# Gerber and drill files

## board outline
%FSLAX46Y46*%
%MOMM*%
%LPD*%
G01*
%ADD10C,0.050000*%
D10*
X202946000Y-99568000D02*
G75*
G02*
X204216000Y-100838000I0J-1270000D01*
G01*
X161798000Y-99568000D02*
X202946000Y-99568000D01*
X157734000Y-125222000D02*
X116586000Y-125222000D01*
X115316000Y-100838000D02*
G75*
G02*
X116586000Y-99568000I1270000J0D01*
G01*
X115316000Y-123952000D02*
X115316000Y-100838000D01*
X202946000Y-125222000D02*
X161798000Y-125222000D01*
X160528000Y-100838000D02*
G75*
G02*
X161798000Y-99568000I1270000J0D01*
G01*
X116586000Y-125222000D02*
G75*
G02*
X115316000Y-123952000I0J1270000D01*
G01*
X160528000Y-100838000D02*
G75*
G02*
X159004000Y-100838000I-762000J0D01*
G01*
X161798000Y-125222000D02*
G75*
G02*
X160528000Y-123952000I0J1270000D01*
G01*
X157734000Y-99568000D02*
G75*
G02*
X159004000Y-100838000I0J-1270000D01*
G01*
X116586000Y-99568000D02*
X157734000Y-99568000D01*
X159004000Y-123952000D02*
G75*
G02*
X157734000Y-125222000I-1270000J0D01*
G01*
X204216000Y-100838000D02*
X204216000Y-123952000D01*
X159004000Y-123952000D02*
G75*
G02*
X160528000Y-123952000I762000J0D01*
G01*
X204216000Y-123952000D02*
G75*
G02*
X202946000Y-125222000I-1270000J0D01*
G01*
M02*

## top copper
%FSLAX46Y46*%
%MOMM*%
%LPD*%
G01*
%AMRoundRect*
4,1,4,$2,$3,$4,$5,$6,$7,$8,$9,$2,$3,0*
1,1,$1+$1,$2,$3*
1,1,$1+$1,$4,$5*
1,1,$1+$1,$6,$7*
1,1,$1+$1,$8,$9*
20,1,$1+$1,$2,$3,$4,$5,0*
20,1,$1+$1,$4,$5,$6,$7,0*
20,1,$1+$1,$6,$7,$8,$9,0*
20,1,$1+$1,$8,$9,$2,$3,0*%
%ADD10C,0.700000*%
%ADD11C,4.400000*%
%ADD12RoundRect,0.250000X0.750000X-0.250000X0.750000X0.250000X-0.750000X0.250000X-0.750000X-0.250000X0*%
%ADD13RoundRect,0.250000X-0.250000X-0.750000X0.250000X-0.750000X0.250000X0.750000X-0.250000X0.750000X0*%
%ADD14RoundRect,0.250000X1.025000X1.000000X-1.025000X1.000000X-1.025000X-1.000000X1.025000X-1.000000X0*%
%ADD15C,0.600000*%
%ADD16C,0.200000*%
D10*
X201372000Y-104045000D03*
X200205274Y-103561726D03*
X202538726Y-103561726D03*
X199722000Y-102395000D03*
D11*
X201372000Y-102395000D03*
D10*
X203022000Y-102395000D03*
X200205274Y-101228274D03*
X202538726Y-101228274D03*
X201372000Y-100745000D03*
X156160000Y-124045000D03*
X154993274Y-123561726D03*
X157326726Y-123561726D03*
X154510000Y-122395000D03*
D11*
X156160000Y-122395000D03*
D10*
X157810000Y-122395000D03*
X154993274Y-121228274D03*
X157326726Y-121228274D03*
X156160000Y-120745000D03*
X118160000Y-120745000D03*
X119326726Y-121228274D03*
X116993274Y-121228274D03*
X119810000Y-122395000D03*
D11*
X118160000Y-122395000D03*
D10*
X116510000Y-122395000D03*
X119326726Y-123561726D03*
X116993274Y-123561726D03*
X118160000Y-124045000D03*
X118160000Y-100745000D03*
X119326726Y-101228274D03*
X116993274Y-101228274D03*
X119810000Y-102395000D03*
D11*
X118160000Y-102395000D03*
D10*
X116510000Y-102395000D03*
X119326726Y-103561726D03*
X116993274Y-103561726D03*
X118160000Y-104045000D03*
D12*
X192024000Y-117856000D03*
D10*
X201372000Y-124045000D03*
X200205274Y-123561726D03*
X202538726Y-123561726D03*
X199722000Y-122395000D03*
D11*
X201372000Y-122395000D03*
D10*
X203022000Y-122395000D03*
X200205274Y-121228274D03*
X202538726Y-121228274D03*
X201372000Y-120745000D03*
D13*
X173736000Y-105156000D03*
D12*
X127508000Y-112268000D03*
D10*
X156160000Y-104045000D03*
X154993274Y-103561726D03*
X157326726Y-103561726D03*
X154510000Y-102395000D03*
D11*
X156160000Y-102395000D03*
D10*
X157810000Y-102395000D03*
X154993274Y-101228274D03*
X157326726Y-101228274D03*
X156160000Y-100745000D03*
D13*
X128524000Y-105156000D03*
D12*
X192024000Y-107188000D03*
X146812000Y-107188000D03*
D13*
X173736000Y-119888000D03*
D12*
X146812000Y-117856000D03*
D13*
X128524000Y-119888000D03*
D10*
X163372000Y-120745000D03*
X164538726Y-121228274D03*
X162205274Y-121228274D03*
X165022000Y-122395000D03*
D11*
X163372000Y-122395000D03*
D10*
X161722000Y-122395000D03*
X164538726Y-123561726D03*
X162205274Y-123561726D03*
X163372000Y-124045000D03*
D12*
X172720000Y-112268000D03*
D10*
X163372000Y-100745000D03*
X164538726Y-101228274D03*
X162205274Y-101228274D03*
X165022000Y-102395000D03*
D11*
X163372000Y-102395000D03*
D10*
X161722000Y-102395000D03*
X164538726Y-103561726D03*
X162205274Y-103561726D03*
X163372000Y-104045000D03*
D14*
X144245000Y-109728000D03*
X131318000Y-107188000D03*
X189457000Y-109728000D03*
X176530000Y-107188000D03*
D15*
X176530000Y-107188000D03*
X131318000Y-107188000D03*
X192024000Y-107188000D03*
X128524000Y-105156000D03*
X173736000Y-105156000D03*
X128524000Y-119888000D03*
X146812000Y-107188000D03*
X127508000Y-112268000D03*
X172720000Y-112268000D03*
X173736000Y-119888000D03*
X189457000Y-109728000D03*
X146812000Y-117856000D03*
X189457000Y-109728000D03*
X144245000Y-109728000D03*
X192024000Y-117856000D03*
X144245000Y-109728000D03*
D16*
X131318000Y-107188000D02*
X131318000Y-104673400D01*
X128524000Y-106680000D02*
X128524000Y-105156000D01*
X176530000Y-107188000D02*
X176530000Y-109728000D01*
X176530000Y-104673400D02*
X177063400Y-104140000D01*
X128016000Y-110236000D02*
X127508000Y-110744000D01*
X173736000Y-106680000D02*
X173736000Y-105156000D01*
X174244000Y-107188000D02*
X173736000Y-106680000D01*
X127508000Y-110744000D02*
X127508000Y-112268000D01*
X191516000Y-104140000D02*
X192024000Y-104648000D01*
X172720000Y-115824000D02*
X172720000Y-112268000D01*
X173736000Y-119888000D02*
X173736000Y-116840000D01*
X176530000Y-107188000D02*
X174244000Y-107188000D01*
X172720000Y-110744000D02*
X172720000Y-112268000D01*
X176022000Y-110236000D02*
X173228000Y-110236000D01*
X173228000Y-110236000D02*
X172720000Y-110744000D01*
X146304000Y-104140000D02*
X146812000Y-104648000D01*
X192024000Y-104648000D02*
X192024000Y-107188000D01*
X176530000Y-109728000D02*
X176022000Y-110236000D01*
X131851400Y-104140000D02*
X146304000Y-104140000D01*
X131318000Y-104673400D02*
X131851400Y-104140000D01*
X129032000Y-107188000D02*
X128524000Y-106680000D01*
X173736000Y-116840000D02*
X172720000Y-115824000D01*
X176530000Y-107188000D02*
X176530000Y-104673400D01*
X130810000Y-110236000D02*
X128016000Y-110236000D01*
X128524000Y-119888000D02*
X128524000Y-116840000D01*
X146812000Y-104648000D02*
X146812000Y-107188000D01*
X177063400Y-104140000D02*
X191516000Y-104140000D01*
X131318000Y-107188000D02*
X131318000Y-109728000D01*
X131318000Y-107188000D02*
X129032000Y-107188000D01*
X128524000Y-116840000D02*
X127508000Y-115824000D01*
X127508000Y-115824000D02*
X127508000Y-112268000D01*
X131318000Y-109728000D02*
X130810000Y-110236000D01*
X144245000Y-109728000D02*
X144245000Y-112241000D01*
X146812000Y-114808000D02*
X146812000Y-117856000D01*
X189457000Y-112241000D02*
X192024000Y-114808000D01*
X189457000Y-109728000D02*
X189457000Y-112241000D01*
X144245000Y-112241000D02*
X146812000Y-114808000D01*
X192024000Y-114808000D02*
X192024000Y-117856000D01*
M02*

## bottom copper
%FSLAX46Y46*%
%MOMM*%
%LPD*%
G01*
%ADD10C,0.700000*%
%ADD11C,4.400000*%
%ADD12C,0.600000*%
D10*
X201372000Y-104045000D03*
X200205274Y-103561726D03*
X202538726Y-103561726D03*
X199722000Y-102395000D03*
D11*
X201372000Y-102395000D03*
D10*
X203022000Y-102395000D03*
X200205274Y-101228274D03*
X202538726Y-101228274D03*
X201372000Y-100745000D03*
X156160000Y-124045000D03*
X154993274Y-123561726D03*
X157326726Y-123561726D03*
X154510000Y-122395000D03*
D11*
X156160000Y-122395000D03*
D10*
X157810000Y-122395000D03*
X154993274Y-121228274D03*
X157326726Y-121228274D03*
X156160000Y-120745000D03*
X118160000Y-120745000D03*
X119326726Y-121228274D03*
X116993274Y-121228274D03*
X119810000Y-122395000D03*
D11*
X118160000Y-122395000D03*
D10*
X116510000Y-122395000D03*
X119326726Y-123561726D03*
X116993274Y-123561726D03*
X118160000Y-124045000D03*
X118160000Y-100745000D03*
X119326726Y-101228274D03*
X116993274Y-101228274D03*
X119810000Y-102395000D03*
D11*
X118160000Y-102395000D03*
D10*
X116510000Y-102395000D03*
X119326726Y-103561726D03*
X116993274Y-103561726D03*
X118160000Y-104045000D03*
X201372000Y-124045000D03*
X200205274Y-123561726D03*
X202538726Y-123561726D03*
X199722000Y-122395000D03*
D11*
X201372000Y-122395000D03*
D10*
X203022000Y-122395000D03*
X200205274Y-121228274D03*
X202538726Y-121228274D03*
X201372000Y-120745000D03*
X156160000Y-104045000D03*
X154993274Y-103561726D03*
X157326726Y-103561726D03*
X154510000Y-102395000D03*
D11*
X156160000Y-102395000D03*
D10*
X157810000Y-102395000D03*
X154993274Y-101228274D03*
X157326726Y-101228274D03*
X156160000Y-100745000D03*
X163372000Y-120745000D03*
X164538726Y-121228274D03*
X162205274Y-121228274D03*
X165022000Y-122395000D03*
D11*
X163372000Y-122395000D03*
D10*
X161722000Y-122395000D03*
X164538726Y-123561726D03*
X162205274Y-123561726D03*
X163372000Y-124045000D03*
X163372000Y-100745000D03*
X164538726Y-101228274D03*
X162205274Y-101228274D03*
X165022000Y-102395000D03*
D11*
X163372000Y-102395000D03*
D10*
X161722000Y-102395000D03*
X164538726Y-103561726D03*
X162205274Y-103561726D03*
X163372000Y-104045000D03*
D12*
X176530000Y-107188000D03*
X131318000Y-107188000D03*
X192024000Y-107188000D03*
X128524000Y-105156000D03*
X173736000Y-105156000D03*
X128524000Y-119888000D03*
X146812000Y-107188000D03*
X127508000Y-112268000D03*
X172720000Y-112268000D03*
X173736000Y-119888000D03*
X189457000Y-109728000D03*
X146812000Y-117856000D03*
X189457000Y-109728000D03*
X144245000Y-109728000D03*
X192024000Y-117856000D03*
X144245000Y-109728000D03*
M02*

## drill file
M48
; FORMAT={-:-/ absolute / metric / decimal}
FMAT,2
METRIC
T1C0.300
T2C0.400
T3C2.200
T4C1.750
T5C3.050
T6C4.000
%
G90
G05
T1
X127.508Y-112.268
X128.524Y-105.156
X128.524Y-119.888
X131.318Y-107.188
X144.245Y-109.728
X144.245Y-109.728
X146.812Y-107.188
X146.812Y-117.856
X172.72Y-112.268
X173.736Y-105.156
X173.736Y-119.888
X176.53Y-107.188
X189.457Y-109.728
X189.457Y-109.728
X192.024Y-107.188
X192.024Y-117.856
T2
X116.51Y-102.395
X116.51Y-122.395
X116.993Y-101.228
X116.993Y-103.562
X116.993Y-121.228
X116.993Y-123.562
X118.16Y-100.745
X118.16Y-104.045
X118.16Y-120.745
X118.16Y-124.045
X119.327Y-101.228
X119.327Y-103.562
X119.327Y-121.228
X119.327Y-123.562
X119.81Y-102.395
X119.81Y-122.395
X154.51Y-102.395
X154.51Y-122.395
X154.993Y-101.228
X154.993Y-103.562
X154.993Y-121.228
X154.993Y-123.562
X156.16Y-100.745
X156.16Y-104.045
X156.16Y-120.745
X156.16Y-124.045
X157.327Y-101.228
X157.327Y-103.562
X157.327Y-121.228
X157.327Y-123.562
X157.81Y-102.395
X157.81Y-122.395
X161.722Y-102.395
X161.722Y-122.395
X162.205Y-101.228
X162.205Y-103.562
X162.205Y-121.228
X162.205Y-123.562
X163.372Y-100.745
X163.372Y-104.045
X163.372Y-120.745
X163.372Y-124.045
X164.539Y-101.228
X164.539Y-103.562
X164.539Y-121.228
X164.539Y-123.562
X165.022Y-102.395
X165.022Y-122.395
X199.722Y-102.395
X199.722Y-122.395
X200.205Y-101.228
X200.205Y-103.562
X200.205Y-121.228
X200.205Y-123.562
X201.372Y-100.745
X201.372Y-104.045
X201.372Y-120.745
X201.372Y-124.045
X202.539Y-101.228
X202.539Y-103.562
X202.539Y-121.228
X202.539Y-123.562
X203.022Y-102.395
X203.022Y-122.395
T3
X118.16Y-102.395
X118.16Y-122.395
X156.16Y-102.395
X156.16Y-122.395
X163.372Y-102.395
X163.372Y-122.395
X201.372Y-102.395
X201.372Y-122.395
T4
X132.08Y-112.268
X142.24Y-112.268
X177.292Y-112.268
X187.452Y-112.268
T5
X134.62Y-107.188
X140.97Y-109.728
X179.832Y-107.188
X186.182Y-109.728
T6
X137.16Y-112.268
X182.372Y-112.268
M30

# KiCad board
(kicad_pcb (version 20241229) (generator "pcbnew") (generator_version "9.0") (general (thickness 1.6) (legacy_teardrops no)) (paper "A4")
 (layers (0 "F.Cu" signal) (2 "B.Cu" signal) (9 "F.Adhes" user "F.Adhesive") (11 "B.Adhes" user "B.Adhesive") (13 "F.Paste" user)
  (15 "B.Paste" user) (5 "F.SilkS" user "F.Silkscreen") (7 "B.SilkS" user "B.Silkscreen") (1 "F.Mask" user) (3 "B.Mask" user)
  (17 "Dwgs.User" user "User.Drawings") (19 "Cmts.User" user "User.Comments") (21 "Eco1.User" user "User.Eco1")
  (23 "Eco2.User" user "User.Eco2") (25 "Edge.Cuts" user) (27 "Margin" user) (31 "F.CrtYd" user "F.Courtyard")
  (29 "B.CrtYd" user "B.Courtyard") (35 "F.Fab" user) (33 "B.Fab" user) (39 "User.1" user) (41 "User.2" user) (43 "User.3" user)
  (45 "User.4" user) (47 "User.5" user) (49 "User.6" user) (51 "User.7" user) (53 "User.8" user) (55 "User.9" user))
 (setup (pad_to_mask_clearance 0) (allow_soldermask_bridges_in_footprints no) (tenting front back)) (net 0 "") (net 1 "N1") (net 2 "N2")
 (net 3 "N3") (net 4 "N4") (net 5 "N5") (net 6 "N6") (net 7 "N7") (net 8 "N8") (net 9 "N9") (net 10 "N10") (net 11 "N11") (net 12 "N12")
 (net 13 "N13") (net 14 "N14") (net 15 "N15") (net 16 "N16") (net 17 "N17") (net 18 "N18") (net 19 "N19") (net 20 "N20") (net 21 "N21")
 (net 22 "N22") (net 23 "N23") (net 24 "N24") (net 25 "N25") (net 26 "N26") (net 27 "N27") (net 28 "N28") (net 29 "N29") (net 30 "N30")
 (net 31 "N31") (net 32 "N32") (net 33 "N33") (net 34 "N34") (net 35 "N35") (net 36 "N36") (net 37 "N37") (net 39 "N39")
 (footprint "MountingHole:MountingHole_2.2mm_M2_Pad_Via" (layer "F.Cu") (at 201.372 102.395 90)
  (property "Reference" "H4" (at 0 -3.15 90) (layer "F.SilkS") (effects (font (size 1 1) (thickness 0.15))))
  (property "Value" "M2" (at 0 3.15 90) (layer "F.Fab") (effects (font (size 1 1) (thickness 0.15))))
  (pad "1" thru_hole circle (at -1.65 0 90) (size 0.7 0.7) (drill 0.4) (layers "*.Cu" "*.Mask") (remove_unused_layers no) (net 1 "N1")
   (zone_connect 2))
  (pad "1" thru_hole circle (at -1.166726 -1.166726 90) (size 0.7 0.7) (drill 0.4) (layers "*.Cu" "*.Mask") (remove_unused_layers no)
   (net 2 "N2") (zone_connect 2))
  (pad "1" thru_hole circle (at -1.166726 1.166726 90) (size 0.7 0.7) (drill 0.4) (layers "*.Cu" "*.Mask") (remove_unused_layers no)
   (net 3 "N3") (zone_connect 2))
  (pad "1" thru_hole circle (at 0 -1.65 90) (size 0.7 0.7) (drill 0.4) (layers "*.Cu" "*.Mask") (remove_unused_layers no) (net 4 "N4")
   (zone_connect 2))
  (pad "1" thru_hole circle (at 0 0 90) (size 4.4 4.4) (drill 2.2) (layers "*.Cu" "*.Mask") (remove_unused_layers no) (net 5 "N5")
   (zone_connect 2))
  (pad "1" thru_hole circle (at 0 1.65 90) (size 0.7 0.7) (drill 0.4) (layers "*.Cu" "*.Mask") (remove_unused_layers no) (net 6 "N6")
   (zone_connect 2))
  (pad "1" thru_hole circle (at 1.166726 -1.166726 90) (size 0.7 0.7) (drill 0.4) (layers "*.Cu" "*.Mask") (remove_unused_layers no)
   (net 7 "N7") (zone_connect 2))
  (pad "1" thru_hole circle (at 1.166726 1.166726 90) (size 0.7 0.7) (drill 0.4) (layers "*.Cu" "*.Mask") (remove_unused_layers no)
   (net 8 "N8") (zone_connect 2))
  (pad "1" thru_hole circle (at 1.65 0 90) (size 0.7 0.7) (drill 0.4) (layers "*.Cu" "*.Mask") (remove_unused_layers no) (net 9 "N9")
   (zone_connect 2)))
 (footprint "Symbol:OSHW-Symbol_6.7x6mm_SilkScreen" (layer "F.Cu") (at 133.096 117.856)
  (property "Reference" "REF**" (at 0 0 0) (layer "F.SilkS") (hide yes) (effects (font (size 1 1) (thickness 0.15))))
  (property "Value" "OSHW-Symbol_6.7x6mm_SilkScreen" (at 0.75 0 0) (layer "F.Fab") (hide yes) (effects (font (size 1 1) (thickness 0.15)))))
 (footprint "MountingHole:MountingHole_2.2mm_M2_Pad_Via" (layer "F.Cu") (at 156.16 122.395 90)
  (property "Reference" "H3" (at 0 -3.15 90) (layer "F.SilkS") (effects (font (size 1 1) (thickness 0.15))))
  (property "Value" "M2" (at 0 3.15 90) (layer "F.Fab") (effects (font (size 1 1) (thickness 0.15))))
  (pad "1" thru_hole circle (at -1.65 0 90) (size 0.7 0.7) (drill 0.4) (layers "*.Cu" "*.Mask") (remove_unused_layers no) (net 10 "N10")
   (zone_connect 2))
  (pad "1" thru_hole circle (at -1.166726 -1.166726 90) (size 0.7 0.7) (drill 0.4) (layers "*.Cu" "*.Mask") (remove_unused_layers no)
   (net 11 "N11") (zone_connect 2))
  (pad "1" thru_hole circle (at -1.166726 1.166726 90) (size 0.7 0.7) (drill 0.4) (layers "*.Cu" "*.Mask") (remove_unused_layers no)
   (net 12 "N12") (zone_connect 2))
  (pad "1" thru_hole circle (at 0 -1.65 90) (size 0.7 0.7) (drill 0.4) (layers "*.Cu" "*.Mask") (remove_unused_layers no) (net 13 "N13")
   (zone_connect 2))
  (pad "1" thru_hole circle (at 0 0 90) (size 4.4 4.4) (drill 2.2) (layers "*.Cu" "*.Mask") (remove_unused_layers no) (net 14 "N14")
   (zone_connect 2))
  (pad "1" thru_hole circle (at 0 1.65 90) (size 0.7 0.7) (drill 0.4) (layers "*.Cu" "*.Mask") (remove_unused_layers no) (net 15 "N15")
   (zone_connect 2))
  (pad "1" thru_hole circle (at 1.166726 -1.166726 90) (size 0.7 0.7) (drill 0.4) (layers "*.Cu" "*.Mask") (remove_unused_layers no)
   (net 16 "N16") (zone_connect 2))
  (pad "1" thru_hole circle (at 1.166726 1.166726 90) (size 0.7 0.7) (drill 0.4) (layers "*.Cu" "*.Mask") (remove_unused_layers no)
   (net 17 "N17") (zone_connect 2))
  (pad "1" thru_hole circle (at 1.65 0 90) (size 0.7 0.7) (drill 0.4) (layers "*.Cu" "*.Mask") (remove_unused_layers no) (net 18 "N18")
   (zone_connect 2)))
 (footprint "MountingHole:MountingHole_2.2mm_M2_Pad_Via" (layer "F.Cu") (at 118.16 122.395 -90)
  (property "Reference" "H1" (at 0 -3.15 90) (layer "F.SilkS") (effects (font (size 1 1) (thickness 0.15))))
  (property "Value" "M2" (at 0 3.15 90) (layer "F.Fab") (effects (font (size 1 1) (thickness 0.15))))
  (pad "1" thru_hole circle (at -1.65 0 270) (size 0.7 0.7) (drill 0.4) (layers "*.Cu" "*.Mask") (remove_unused_layers no) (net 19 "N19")
   (zone_connect 2))
  (pad "1" thru_hole circle (at -1.166726 -1.166726 270) (size 0.7 0.7) (drill 0.4) (layers "*.Cu" "*.Mask") (remove_unused_layers no)
   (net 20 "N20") (zone_connect 2))
  (pad "1" thru_hole circle (at -1.166726 1.166726 270) (size 0.7 0.7) (drill 0.4) (layers "*.Cu" "*.Mask") (remove_unused_layers no)
   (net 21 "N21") (zone_connect 2))
  (pad "1" thru_hole circle (at 0 -1.65 270) (size 0.7 0.7) (drill 0.4) (layers "*.Cu" "*.Mask") (remove_unused_layers no) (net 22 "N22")
   (zone_connect 2))
  (pad "1" thru_hole circle (at 0 0 270) (size 4.4 4.4) (drill 2.2) (layers "*.Cu" "*.Mask") (remove_unused_layers no) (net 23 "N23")
   (zone_connect 2))
  (pad "1" thru_hole circle (at 0 1.65 270) (size 0.7 0.7) (drill 0.4) (layers "*.Cu" "*.Mask") (remove_unused_layers no) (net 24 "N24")
   (zone_connect 2))
  (pad "1" thru_hole circle (at 1.166726 -1.166726 270) (size 0.7 0.7) (drill 0.4) (layers "*.Cu" "*.Mask") (remove_unused_layers no)
   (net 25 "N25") (zone_connect 2))
  (pad "1" thru_hole circle (at 1.166726 1.166726 270) (size 0.7 0.7) (drill 0.4) (layers "*.Cu" "*.Mask") (remove_unused_layers no)
   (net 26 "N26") (zone_connect 2))
  (pad "1" thru_hole circle (at 1.65 0 270) (size 0.7 0.7) (drill 0.4) (layers "*.Cu" "*.Mask") (remove_unused_layers no) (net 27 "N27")
   (zone_connect 2)))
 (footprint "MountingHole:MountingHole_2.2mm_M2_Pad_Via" (layer "F.Cu") (at 118.16 102.395 -90)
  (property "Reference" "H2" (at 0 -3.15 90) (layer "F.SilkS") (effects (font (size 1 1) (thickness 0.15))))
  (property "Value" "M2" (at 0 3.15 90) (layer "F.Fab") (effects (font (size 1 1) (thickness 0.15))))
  (pad "1" thru_hole circle (at -1.65 0 270) (size 0.7 0.7) (drill 0.4) (layers "*.Cu" "*.Mask") (remove_unused_layers no) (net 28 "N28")
   (zone_connect 2))
  (pad "1" thru_hole circle (at -1.166726 -1.166726 270) (size 0.7 0.7) (drill 0.4) (layers "*.Cu" "*.Mask") (remove_unused_layers no)
   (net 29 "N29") (zone_connect 2))
  (pad "1" thru_hole circle (at -1.166726 1.166726 270) (size 0.7 0.7) (drill 0.4) (layers "*.Cu" "*.Mask") (remove_unused_layers no)
   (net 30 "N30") (zone_connect 2))
  (pad "1" thru_hole circle (at 0 -1.65 270) (size 0.7 0.7) (drill 0.4) (layers "*.Cu" "*.Mask") (remove_unused_layers no) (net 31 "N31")
   (zone_connect 2))
  (pad "1" thru_hole circle (at 0 0 270) (size 4.4 4.4) (drill 2.2) (layers "*.Cu" "*.Mask") (remove_unused_layers no) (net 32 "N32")
   (zone_connect 2))
  (pad "1" thru_hole circle (at 0 1.65 270) (size 0.7 0.7) (drill 0.4) (layers "*.Cu" "*.Mask") (remove_unused_layers no) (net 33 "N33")
   (zone_connect 2))
  (pad "1" thru_hole circle (at 1.166726 -1.166726 270) (size 0.7 0.7) (drill 0.4) (layers "*.Cu" "*.Mask") (remove_unused_layers no)
   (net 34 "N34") (zone_connect 2))
  (pad "1" thru_hole circle (at 1.166726 1.166726 270) (size 0.7 0.7) (drill 0.4) (layers "*.Cu" "*.Mask") (remove_unused_layers no)
   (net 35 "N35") (zone_connect 2))
  (pad "1" thru_hole circle (at 1.65 0 270) (size 0.7 0.7) (drill 0.4) (layers "*.Cu" "*.Mask") (remove_unused_layers no) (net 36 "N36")
   (zone_connect 2)))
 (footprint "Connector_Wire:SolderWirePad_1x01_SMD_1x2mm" (layer "F.Cu") (at 192.024 117.856 90)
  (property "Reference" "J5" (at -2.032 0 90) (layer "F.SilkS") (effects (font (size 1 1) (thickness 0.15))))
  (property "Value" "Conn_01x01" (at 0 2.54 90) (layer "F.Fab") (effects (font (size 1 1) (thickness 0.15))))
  (pad "1" smd roundrect (at 0 0 90) (size 1 2) (layers "F.Cu" "F.Mask" "F.Paste") (roundrect_rratio 0.25) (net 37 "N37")))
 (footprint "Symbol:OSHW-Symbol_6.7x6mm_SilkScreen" (layer "F.Cu") (at 178.308 117.856)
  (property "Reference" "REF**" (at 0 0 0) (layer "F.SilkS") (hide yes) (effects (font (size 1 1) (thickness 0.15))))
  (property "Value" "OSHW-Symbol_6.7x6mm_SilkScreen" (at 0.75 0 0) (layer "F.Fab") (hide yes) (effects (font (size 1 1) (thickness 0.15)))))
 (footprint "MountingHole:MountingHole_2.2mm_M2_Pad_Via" (layer "F.Cu") (at 201.372 122.395 90)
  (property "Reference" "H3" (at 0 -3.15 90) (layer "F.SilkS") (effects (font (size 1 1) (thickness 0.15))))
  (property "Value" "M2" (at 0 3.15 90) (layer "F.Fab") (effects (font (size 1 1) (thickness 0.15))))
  (pad "1" thru_hole circle (at -1.65 0 90) (size 0.7 0.7) (drill 0.4) (layers "*.Cu" "*.Mask") (remove_unused_layers no) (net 10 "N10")
   (zone_connect 2))
  (pad "1" thru_hole circle (at -1.166726 -1.166726 90) (size 0.7 0.7) (drill 0.4) (layers "*.Cu" "*.Mask") (remove_unused_layers no)
   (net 11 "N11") (zone_connect 2))
  (pad "1" thru_hole circle (at -1.166726 1.166726 90) (size 0.7 0.7) (drill 0.4) (layers "*.Cu" "*.Mask") (remove_unused_layers no)
   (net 12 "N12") (zone_connect 2))
  (pad "1" thru_hole circle (at 0 -1.65 90) (size 0.7 0.7) (drill 0.4) (layers "*.Cu" "*.Mask") (remove_unused_layers no) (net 13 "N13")
   (zone_connect 2))
  (pad "1" thru_hole circle (at 0 0 90) (size 4.4 4.4) (drill 2.2) (layers "*.Cu" "*.Mask") (remove_unused_layers no) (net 14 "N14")
   (zone_connect 2))
  (pad "1" thru_hole circle (at 0 1.65 90) (size 0.7 0.7) (drill 0.4) (layers "*.Cu" "*.Mask") (remove_unused_layers no) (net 15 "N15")
   (zone_connect 2))
  (pad "1" thru_hole circle (at 1.166726 -1.166726 90) (size 0.7 0.7) (drill 0.4) (layers "*.Cu" "*.Mask") (remove_unused_layers no)
   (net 16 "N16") (zone_connect 2))
  (pad "1" thru_hole circle (at 1.166726 1.166726 90) (size 0.7 0.7) (drill 0.4) (layers "*.Cu" "*.Mask") (remove_unused_layers no)
   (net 17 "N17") (zone_connect 2))
  (pad "1" thru_hole circle (at 1.65 0 90) (size 0.7 0.7) (drill 0.4) (layers "*.Cu" "*.Mask") (remove_unused_layers no) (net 18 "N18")
   (zone_connect 2)))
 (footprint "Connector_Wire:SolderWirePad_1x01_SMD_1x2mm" (layer "F.Cu") (at 173.736 105.156)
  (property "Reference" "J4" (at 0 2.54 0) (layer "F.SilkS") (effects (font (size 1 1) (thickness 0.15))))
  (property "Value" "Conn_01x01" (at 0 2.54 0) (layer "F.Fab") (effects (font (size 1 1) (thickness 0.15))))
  (pad "1" smd roundrect (at 0 0) (size 1 2) (layers "F.Cu" "F.Mask" "F.Paste") (roundrect_rratio 0.25) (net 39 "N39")))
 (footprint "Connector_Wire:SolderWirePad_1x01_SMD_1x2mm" (layer "F.Cu") (at 127.508 112.268 90)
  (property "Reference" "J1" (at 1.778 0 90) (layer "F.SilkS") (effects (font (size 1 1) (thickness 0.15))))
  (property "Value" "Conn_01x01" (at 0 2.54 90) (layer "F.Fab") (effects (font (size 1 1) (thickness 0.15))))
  (pad "1" smd roundrect (at 0 0 90) (size 1 2) (layers "F.Cu" "F.Mask" "F.Paste") (roundrect_rratio 0.25) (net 39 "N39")))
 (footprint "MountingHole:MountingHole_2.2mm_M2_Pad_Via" (layer "F.Cu") (at 156.16 102.395 90)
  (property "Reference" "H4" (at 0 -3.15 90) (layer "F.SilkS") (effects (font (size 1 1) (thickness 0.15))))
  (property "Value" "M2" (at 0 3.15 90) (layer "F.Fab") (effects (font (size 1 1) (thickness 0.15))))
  (pad "1" thru_hole circle (at -1.65 0 90) (size 0.7 0.7) (drill 0.4) (layers "*.Cu" "*.Mask") (remove_unused_layers no) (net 1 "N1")
   (zone_connect 2))
  (pad "1" thru_hole circle (at -1.166726 -1.166726 90) (size 0.7 0.7) (drill 0.4) (layers "*.Cu" "*.Mask") (remove_unused_layers no)
   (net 2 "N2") (zone_connect 2))
  (pad "1" thru_hole circle (at -1.166726 1.166726 90) (size 0.7 0.7) (drill 0.4) (layers "*.Cu" "*.Mask") (remove_unused_layers no)
   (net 3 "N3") (zone_connect 2))
  (pad "1" thru_hole circle (at 0 -1.65 90) (size 0.7 0.7) (drill 0.4) (layers "*.Cu" "*.Mask") (remove_unused_layers no) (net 4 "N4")
   (zone_connect 2))
  (pad "1" thru_hole circle (at 0 0 90) (size 4.4 4.4) (drill 2.2) (layers "*.Cu" "*.Mask") (remove_unused_layers no) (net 5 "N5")
   (zone_connect 2))
  (pad "1" thru_hole circle (at 0 1.65 90) (size 0.7 0.7) (drill 0.4) (layers "*.Cu" "*.Mask") (remove_unused_layers no) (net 6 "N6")
   (zone_connect 2))
  (pad "1" thru_hole circle (at 1.166726 -1.166726 90) (size 0.7 0.7) (drill 0.4) (layers "*.Cu" "*.Mask") (remove_unused_layers no)
   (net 7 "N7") (zone_connect 2))
  (pad "1" thru_hole circle (at 1.166726 1.166726 90) (size 0.7 0.7) (drill 0.4) (layers "*.Cu" "*.Mask") (remove_unused_layers no)
   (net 8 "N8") (zone_connect 2))
  (pad "1" thru_hole circle (at 1.65 0 90) (size 0.7 0.7) (drill 0.4) (layers "*.Cu" "*.Mask") (remove_unused_layers no) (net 9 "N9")
   (zone_connect 2)))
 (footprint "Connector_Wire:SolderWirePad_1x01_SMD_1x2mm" (layer "F.Cu") (at 128.524 105.156)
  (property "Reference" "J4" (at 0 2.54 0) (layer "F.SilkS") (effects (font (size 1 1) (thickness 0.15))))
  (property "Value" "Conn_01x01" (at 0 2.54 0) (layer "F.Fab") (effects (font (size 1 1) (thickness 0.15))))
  (pad "1" smd roundrect (at 0 0) (size 1 2) (layers "F.Cu" "F.Mask" "F.Paste") (roundrect_rratio 0.25) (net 39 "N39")))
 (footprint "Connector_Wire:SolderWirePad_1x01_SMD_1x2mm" (layer "F.Cu") (at 192.024 107.188 90)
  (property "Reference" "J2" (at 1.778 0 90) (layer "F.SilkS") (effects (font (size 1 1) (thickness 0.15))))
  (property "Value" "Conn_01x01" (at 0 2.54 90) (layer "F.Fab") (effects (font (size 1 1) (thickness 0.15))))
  (pad "1" smd roundrect (at 0 0 90) (size 1 2) (layers "F.Cu" "F.Mask" "F.Paste") (roundrect_rratio 0.25) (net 39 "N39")))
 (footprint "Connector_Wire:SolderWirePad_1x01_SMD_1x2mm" (layer "F.Cu") (at 146.812 107.188 90)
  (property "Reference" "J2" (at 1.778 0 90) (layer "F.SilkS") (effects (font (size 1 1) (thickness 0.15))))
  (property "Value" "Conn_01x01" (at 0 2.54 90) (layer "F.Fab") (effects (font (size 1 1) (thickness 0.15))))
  (pad "1" smd roundrect (at 0 0 90) (size 1 2) (layers "F.Cu" "F.Mask" "F.Paste") (roundrect_rratio 0.25) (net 39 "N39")))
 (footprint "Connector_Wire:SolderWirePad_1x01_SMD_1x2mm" (layer "F.Cu") (at 173.736 119.888)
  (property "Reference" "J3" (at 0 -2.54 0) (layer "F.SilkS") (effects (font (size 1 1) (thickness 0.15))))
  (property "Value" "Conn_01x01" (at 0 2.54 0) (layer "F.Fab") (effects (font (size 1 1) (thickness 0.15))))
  (pad "1" smd roundrect (at 0 0) (size 1 2) (layers "F.Cu" "F.Mask" "F.Paste") (roundrect_rratio 0.25) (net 39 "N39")))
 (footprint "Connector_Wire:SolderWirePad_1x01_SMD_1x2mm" (layer "F.Cu") (at 146.812 117.856 90)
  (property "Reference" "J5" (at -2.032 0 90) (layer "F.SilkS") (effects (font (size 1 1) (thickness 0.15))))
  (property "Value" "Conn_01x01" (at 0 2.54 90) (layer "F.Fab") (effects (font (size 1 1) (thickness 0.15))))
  (pad "1" smd roundrect (at 0 0 90) (size 1 2) (layers "F.Cu" "F.Mask" "F.Paste") (roundrect_rratio 0.25) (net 37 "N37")))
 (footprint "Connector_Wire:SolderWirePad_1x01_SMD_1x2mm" (layer "F.Cu") (at 128.524 119.888)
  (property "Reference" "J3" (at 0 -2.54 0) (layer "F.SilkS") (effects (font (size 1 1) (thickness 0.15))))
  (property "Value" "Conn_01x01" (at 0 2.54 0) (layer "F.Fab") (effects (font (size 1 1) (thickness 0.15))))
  (pad "1" smd roundrect (at 0 0) (size 1 2) (layers "F.Cu" "F.Mask" "F.Paste") (roundrect_rratio 0.25) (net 39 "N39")))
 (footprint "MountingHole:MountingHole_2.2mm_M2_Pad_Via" (layer "F.Cu") (at 163.372 122.395 -90)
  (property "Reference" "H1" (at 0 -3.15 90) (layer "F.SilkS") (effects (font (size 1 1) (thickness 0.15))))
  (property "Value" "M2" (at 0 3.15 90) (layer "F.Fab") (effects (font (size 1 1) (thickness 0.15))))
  (pad "1" thru_hole circle (at -1.65 0 270) (size 0.7 0.7) (drill 0.4) (layers "*.Cu" "*.Mask") (remove_unused_layers no) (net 19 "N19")
   (zone_connect 2))
  (pad "1" thru_hole circle (at -1.166726 -1.166726 270) (size 0.7 0.7) (drill 0.4) (layers "*.Cu" "*.Mask") (remove_unused_layers no)
   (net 20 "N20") (zone_connect 2))
  (pad "1" thru_hole circle (at -1.166726 1.166726 270) (size 0.7 0.7) (drill 0.4) (layers "*.Cu" "*.Mask") (remove_unused_layers no)
   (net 21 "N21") (zone_connect 2))
  (pad "1" thru_hole circle (at 0 -1.65 270) (size 0.7 0.7) (drill 0.4) (layers "*.Cu" "*.Mask") (remove_unused_layers no) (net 22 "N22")
   (zone_connect 2))
  (pad "1" thru_hole circle (at 0 0 270) (size 4.4 4.4) (drill 2.2) (layers "*.Cu" "*.Mask") (remove_unused_layers no) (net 23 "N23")
   (zone_connect 2))
  (pad "1" thru_hole circle (at 0 1.65 270) (size 0.7 0.7) (drill 0.4) (layers "*.Cu" "*.Mask") (remove_unused_layers no) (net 24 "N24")
   (zone_connect 2))
  (pad "1" thru_hole circle (at 1.166726 -1.166726 270) (size 0.7 0.7) (drill 0.4) (layers "*.Cu" "*.Mask") (remove_unused_layers no)
   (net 25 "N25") (zone_connect 2))
  (pad "1" thru_hole circle (at 1.166726 1.166726 270) (size 0.7 0.7) (drill 0.4) (layers "*.Cu" "*.Mask") (remove_unused_layers no)
   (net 26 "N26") (zone_connect 2))
  (pad "1" thru_hole circle (at 1.65 0 270) (size 0.7 0.7) (drill 0.4) (layers "*.Cu" "*.Mask") (remove_unused_layers no) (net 27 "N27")
   (zone_connect 2)))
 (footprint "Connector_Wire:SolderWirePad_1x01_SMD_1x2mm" (layer "F.Cu") (at 172.72 112.268 90)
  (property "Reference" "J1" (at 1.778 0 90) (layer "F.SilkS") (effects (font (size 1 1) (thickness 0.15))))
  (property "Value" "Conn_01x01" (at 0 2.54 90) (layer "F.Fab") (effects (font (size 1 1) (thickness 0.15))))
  (pad "1" smd roundrect (at 0 0 90) (size 1 2) (layers "F.Cu" "F.Mask" "F.Paste") (roundrect_rratio 0.25) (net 39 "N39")))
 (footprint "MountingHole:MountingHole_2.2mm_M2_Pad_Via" (layer "F.Cu") (at 163.372 102.395 -90)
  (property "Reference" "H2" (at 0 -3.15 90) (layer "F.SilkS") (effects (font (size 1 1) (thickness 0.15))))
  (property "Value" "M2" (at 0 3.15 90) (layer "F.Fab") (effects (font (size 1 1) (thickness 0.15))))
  (pad "1" thru_hole circle (at -1.65 0 270) (size 0.7 0.7) (drill 0.4) (layers "*.Cu" "*.Mask") (remove_unused_layers no) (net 28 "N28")
   (zone_connect 2))
  (pad "1" thru_hole circle (at -1.166726 -1.166726 270) (size 0.7 0.7) (drill 0.4) (layers "*.Cu" "*.Mask") (remove_unused_layers no)
   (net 29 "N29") (zone_connect 2))
  (pad "1" thru_hole circle (at -1.166726 1.166726 270) (size 0.7 0.7) (drill 0.4) (layers "*.Cu" "*.Mask") (remove_unused_layers no)
   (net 30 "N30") (zone_connect 2))
  (pad "1" thru_hole circle (at 0 -1.65 270) (size 0.7 0.7) (drill 0.4) (layers "*.Cu" "*.Mask") (remove_unused_layers no) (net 31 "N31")
   (zone_connect 2))
  (pad "1" thru_hole circle (at 0 0 270) (size 4.4 4.4) (drill 2.2) (layers "*.Cu" "*.Mask") (remove_unused_layers no) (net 32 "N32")
   (zone_connect 2))
  (pad "1" thru_hole circle (at 0 1.65 270) (size 0.7 0.7) (drill 0.4) (layers "*.Cu" "*.Mask") (remove_unused_layers no) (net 33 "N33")
   (zone_connect 2))
  (pad "1" thru_hole circle (at 1.166726 -1.166726 270) (size 0.7 0.7) (drill 0.4) (layers "*.Cu" "*.Mask") (remove_unused_layers no)
   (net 34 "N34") (zone_connect 2))
  (pad "1" thru_hole circle (at 1.166726 1.166726 270) (size 0.7 0.7) (drill 0.4) (layers "*.Cu" "*.Mask") (remove_unused_layers no)
   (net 35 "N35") (zone_connect 2))
  (pad "1" thru_hole circle (at 1.65 0 270) (size 0.7 0.7) (drill 0.4) (layers "*.Cu" "*.Mask") (remove_unused_layers no) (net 36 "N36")
   (zone_connect 2)))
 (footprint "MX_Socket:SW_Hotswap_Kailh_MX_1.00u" (layer "B.Cu") (at 137.16 112.268 180)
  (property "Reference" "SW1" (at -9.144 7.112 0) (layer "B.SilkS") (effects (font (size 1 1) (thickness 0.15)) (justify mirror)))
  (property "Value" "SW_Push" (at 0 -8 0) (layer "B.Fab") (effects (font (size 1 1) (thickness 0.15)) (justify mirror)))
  (pad "" np_thru_hole circle (at -5.08 0 180) (size 1.75 1.75) (drill 1.75) (layers "*.Cu" "*.Mask"))
  (pad "" np_thru_hole circle (at -3.81 2.54 180) (size 3.05 3.05) (drill 3.05) (layers "*.Cu" "*.Mask"))
  (pad "" np_thru_hole circle (at 0 0 180) (size 4 4) (drill 4) (layers "*.Cu" "*.Mask"))
  (pad "" np_thru_hole circle (at 2.54 5.08 180) (size 3.05 3.05) (drill 3.05) (layers "*.Cu" "*.Mask"))
  (pad "" np_thru_hole circle (at 5.08 0 180) (size 1.75 1.75) (drill 1.75) (layers "*.Cu" "*.Mask"))
  (pad "1" smd roundrect (at -7.085 2.54 180) (size 2.55 2.5) (layers "F.Cu" "F.Mask" "F.Paste") (roundrect_rratio 0.1) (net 37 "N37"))
  (pad "2" smd roundrect (at 5.842 5.08 180) (size 2.55 2.5) (layers "F.Cu" "F.Mask" "F.Paste") (roundrect_rratio 0.1) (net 39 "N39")))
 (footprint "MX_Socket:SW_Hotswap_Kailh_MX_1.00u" (layer "B.Cu") (at 182.372 112.268 180)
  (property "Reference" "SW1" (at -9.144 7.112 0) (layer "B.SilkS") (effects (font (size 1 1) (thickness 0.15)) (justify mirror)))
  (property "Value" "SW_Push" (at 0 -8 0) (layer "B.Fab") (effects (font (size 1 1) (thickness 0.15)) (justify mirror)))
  (pad "" np_thru_hole circle (at -5.08 0 180) (size 1.75 1.75) (drill 1.75) (layers "*.Cu" "*.Mask"))
  (pad "" np_thru_hole circle (at -3.81 2.54 180) (size 3.05 3.05) (drill 3.05) (layers "*.Cu" "*.Mask"))
  (pad "" np_thru_hole circle (at 0 0 180) (size 4 4) (drill 4) (layers "*.Cu" "*.Mask"))
  (pad "" np_thru_hole circle (at 2.54 5.08 180) (size 3.05 3.05) (drill 3.05) (layers "*.Cu" "*.Mask"))
  (pad "" np_thru_hole circle (at 5.08 0 180) (size 1.75 1.75) (drill 1.75) (layers "*.Cu" "*.Mask"))
  (pad "1" smd roundrect (at -7.085 2.54 180) (size 2.55 2.5) (layers "F.Cu" "F.Mask" "F.Paste") (roundrect_rratio 0.1) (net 37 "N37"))
  (pad "2" smd roundrect (at 5.842 5.08 180) (size 2.55 2.5) (layers "F.Cu" "F.Mask" "F.Paste") (roundrect_rratio 0.1) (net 39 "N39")))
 (gr_arc (start 202.946 99.568) (mid 203.844026 99.939974) (end 204.216 100.838) (stroke (width 0.05) (type default)) (layer "Edge.Cuts"))
 (gr_line (start 161.798 99.568) (end 202.946 99.568) (stroke (width 0.05) (type default)) (layer "Edge.Cuts"))
 (gr_line (start 157.734 125.222) (end 116.586 125.222) (stroke (width 0.05) (type default)) (layer "Edge.Cuts"))
 (gr_arc (start 115.316 100.838) (mid 115.687974 99.939974) (end 116.586 99.568) (stroke (width 0.05) (type default)) (layer "Edge.Cuts"))
 (gr_line (start 115.316 123.952) (end 115.316 100.838) (stroke (width 0.05) (type default)) (layer "Edge.Cuts"))
 (gr_line (start 202.946 125.222) (end 161.798 125.222) (stroke (width 0.05) (type default)) (layer "Edge.Cuts"))
 (gr_arc (start 160.528 100.838) (mid 160.899974 99.939974) (end 161.798 99.568) (stroke (width 0.05) (type default)) (layer "Edge.Cuts"))
 (gr_arc (start 116.586 125.222) (mid 115.687974 124.850026) (end 115.316 123.952) (stroke (width 0.05) (type default)) (layer "Edge.Cuts"))
 (gr_arc (start 160.528 100.838) (mid 159.766 101.6) (end 159.004 100.838) (stroke (width 0.05) (type default)) (layer "Edge.Cuts"))
 (gr_arc (start 161.798 125.222) (mid 160.899974 124.850026) (end 160.528 123.952) (stroke (width 0.05) (type default)) (layer "Edge.Cuts"))
 (gr_arc (start 157.734 99.568) (mid 158.632026 99.939974) (end 159.004 100.838) (stroke (width 0.05) (type default)) (layer "Edge.Cuts"))
 (gr_line (start 116.586 99.568) (end 157.734 99.568) (stroke (width 0.05) (type default)) (layer "Edge.Cuts"))
 (gr_arc (start 159.004 123.952) (mid 158.632026 124.850026) (end 157.734 125.222) (stroke (width 0.05) (type default)) (layer "Edge.Cuts"))
 (gr_line (start 204.216 100.838) (end 204.216 123.952) (stroke (width 0.05) (type default)) (layer "Edge.Cuts"))
 (gr_arc (start 159.004 123.952) (mid 159.766 123.19) (end 160.528 123.952) (stroke (width 0.05) (type default)) (layer "Edge.Cuts"))
 (gr_arc (start 204.216 123.952) (mid 203.844026 124.850026) (end 202.946 125.222) (stroke (width 0.05) (type default)) (layer "Edge.Cuts"))
 (segment (start 131.318 107.188) (end 131.318 104.6734) (width 0.2) (layer "F.Cu") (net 39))
 (segment (start 128.524 106.68) (end 128.524 105.156) (width 0.2) (layer "F.Cu") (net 39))
 (segment (start 176.53 107.188) (end 176.53 109.728) (width 0.2) (layer "F.Cu") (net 39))
 (segment (start 176.53 104.6734) (end 177.0634 104.14) (width 0.2) (layer "F.Cu") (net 39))
 (segment (start 128.016 110.236) (end 127.508 110.744) (width 0.2) (layer "F.Cu") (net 39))
 (segment (start 173.736 106.68) (end 173.736 105.156) (width 0.2) (layer "F.Cu") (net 39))
 (segment (start 174.244 107.188) (end 173.736 106.68) (width 0.2) (layer "F.Cu") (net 39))
 (segment (start 127.508 110.744) (end 127.508 112.268) (width 0.2) (layer "F.Cu") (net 39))
 (segment (start 191.516 104.14) (end 192.024 104.648) (width 0.2) (layer "F.Cu") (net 39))
 (segment (start 172.72 115.824) (end 172.72 112.268) (width 0.2) (layer "F.Cu") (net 39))
 (segment (start 173.736 119.888) (end 173.736 116.84) (width 0.2) (layer "F.Cu") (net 39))
 (segment (start 176.53 107.188) (end 174.244 107.188) (width 0.2) (layer "F.Cu") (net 39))
 (segment (start 172.72 110.744) (end 172.72 112.268) (width 0.2) (layer "F.Cu") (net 39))
 (segment (start 176.022 110.236) (end 173.228 110.236) (width 0.2) (layer "F.Cu") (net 39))
 (segment (start 173.228 110.236) (end 172.72 110.744) (width 0.2) (layer "F.Cu") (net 39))
 (segment (start 146.304 104.14) (end 146.812 104.648) (width 0.2) (layer "F.Cu") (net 39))
 (segment (start 192.024 104.648) (end 192.024 107.188) (width 0.2) (layer "F.Cu") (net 39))
 (segment (start 176.53 109.728) (end 176.022 110.236) (width 0.2) (layer "F.Cu") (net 39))
 (segment (start 131.8514 104.14) (end 146.304 104.14) (width 0.2) (layer "F.Cu") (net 39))
 (segment (start 131.318 104.6734) (end 131.8514 104.14) (width 0.2) (layer "F.Cu") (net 39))
 (segment (start 129.032 107.188) (end 128.524 106.68) (width 0.2) (layer "F.Cu") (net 39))
 (segment (start 173.736 116.84) (end 172.72 115.824) (width 0.2) (layer "F.Cu") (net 39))
 (segment (start 176.53 107.188) (end 176.53 104.6734) (width 0.2) (layer "F.Cu") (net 39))
 (segment (start 130.81 110.236) (end 128.016 110.236) (width 0.2) (layer "F.Cu") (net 39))
 (segment (start 128.524 119.888) (end 128.524 116.84) (width 0.2) (layer "F.Cu") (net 39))
 (segment (start 146.812 104.648) (end 146.812 107.188) (width 0.2) (layer "F.Cu") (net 39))
 (segment (start 177.0634 104.14) (end 191.516 104.14) (width 0.2) (layer "F.Cu") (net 39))
 (segment (start 131.318 107.188) (end 131.318 109.728) (width 0.2) (layer "F.Cu") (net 39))
 (segment (start 131.318 107.188) (end 129.032 107.188) (width 0.2) (layer "F.Cu") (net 39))
 (segment (start 128.524 116.84) (end 127.508 115.824) (width 0.2) (layer "F.Cu") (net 39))
 (segment (start 127.508 115.824) (end 127.508 112.268) (width 0.2) (layer "F.Cu") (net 39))
 (segment (start 131.318 109.728) (end 130.81 110.236) (width 0.2) (layer "F.Cu") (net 39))
 (via (at 176.53 107.188) (size 0.6) (drill 0.3) (layers "F.Cu" "B.Cu") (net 39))
 (via (at 131.318 107.188) (size 0.6) (drill 0.3) (layers "F.Cu" "B.Cu") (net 39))
 (via (at 192.024 107.188) (size 0.6) (drill 0.3) (layers "F.Cu" "B.Cu") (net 39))
 (via (at 128.524 105.156) (size 0.6) (drill 0.3) (layers "F.Cu" "B.Cu") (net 39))
 (via (at 173.736 105.156) (size 0.6) (drill 0.3) (layers "F.Cu" "B.Cu") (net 39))
 (via (at 128.524 119.888) (size 0.6) (drill 0.3) (layers "F.Cu" "B.Cu") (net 39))
 (via (at 146.812 107.188) (size 0.6) (drill 0.3) (layers "F.Cu" "B.Cu") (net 39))
 (via (at 127.508 112.268) (size 0.6) (drill 0.3) (layers "F.Cu" "B.Cu") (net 39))
 (via (at 172.72 112.268) (size 0.6) (drill 0.3) (layers "F.Cu" "B.Cu") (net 39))
 (via (at 173.736 119.888) (size 0.6) (drill 0.3) (layers "F.Cu" "B.Cu") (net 39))
 (segment (start 144.245 109.728) (end 144.245 112.241) (width 0.2) (layer "F.Cu") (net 37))
 (segment (start 146.812 114.808) (end 146.812 117.856) (width 0.2) (layer "F.Cu") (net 37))
 (segment (start 189.457 112.241) (end 192.024 114.808) (width 0.2) (layer "F.Cu") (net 37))
 (segment (start 189.457 109.728) (end 189.457 112.241) (width 0.2) (layer "F.Cu") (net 37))
 (segment (start 144.245 112.241) (end 146.812 114.808) (width 0.2) (layer "F.Cu") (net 37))
 (segment (start 192.024 114.808) (end 192.024 117.856) (width 0.2) (layer "F.Cu") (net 37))
 (via (at 189.457 109.728) (size 0.6) (drill 0.3) (layers "F.Cu" "B.Cu") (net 37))
 (via (at 146.812 117.856) (size 0.6) (drill 0.3) (layers "F.Cu" "B.Cu") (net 37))
 (via (at 189.457 109.728) (size 0.6) (drill 0.3) (layers "F.Cu" "B.Cu") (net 37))
 (via (at 144.245 109.728) (size 0.6) (drill 0.3) (layers "F.Cu" "B.Cu") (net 37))
 (via (at 192.024 117.856) (size 0.6) (drill 0.3) (layers "F.Cu" "B.Cu") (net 37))
 (via (at 144.245 109.728) (size 0.6) (drill 0.3) (layers "F.Cu" "B.Cu") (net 37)))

